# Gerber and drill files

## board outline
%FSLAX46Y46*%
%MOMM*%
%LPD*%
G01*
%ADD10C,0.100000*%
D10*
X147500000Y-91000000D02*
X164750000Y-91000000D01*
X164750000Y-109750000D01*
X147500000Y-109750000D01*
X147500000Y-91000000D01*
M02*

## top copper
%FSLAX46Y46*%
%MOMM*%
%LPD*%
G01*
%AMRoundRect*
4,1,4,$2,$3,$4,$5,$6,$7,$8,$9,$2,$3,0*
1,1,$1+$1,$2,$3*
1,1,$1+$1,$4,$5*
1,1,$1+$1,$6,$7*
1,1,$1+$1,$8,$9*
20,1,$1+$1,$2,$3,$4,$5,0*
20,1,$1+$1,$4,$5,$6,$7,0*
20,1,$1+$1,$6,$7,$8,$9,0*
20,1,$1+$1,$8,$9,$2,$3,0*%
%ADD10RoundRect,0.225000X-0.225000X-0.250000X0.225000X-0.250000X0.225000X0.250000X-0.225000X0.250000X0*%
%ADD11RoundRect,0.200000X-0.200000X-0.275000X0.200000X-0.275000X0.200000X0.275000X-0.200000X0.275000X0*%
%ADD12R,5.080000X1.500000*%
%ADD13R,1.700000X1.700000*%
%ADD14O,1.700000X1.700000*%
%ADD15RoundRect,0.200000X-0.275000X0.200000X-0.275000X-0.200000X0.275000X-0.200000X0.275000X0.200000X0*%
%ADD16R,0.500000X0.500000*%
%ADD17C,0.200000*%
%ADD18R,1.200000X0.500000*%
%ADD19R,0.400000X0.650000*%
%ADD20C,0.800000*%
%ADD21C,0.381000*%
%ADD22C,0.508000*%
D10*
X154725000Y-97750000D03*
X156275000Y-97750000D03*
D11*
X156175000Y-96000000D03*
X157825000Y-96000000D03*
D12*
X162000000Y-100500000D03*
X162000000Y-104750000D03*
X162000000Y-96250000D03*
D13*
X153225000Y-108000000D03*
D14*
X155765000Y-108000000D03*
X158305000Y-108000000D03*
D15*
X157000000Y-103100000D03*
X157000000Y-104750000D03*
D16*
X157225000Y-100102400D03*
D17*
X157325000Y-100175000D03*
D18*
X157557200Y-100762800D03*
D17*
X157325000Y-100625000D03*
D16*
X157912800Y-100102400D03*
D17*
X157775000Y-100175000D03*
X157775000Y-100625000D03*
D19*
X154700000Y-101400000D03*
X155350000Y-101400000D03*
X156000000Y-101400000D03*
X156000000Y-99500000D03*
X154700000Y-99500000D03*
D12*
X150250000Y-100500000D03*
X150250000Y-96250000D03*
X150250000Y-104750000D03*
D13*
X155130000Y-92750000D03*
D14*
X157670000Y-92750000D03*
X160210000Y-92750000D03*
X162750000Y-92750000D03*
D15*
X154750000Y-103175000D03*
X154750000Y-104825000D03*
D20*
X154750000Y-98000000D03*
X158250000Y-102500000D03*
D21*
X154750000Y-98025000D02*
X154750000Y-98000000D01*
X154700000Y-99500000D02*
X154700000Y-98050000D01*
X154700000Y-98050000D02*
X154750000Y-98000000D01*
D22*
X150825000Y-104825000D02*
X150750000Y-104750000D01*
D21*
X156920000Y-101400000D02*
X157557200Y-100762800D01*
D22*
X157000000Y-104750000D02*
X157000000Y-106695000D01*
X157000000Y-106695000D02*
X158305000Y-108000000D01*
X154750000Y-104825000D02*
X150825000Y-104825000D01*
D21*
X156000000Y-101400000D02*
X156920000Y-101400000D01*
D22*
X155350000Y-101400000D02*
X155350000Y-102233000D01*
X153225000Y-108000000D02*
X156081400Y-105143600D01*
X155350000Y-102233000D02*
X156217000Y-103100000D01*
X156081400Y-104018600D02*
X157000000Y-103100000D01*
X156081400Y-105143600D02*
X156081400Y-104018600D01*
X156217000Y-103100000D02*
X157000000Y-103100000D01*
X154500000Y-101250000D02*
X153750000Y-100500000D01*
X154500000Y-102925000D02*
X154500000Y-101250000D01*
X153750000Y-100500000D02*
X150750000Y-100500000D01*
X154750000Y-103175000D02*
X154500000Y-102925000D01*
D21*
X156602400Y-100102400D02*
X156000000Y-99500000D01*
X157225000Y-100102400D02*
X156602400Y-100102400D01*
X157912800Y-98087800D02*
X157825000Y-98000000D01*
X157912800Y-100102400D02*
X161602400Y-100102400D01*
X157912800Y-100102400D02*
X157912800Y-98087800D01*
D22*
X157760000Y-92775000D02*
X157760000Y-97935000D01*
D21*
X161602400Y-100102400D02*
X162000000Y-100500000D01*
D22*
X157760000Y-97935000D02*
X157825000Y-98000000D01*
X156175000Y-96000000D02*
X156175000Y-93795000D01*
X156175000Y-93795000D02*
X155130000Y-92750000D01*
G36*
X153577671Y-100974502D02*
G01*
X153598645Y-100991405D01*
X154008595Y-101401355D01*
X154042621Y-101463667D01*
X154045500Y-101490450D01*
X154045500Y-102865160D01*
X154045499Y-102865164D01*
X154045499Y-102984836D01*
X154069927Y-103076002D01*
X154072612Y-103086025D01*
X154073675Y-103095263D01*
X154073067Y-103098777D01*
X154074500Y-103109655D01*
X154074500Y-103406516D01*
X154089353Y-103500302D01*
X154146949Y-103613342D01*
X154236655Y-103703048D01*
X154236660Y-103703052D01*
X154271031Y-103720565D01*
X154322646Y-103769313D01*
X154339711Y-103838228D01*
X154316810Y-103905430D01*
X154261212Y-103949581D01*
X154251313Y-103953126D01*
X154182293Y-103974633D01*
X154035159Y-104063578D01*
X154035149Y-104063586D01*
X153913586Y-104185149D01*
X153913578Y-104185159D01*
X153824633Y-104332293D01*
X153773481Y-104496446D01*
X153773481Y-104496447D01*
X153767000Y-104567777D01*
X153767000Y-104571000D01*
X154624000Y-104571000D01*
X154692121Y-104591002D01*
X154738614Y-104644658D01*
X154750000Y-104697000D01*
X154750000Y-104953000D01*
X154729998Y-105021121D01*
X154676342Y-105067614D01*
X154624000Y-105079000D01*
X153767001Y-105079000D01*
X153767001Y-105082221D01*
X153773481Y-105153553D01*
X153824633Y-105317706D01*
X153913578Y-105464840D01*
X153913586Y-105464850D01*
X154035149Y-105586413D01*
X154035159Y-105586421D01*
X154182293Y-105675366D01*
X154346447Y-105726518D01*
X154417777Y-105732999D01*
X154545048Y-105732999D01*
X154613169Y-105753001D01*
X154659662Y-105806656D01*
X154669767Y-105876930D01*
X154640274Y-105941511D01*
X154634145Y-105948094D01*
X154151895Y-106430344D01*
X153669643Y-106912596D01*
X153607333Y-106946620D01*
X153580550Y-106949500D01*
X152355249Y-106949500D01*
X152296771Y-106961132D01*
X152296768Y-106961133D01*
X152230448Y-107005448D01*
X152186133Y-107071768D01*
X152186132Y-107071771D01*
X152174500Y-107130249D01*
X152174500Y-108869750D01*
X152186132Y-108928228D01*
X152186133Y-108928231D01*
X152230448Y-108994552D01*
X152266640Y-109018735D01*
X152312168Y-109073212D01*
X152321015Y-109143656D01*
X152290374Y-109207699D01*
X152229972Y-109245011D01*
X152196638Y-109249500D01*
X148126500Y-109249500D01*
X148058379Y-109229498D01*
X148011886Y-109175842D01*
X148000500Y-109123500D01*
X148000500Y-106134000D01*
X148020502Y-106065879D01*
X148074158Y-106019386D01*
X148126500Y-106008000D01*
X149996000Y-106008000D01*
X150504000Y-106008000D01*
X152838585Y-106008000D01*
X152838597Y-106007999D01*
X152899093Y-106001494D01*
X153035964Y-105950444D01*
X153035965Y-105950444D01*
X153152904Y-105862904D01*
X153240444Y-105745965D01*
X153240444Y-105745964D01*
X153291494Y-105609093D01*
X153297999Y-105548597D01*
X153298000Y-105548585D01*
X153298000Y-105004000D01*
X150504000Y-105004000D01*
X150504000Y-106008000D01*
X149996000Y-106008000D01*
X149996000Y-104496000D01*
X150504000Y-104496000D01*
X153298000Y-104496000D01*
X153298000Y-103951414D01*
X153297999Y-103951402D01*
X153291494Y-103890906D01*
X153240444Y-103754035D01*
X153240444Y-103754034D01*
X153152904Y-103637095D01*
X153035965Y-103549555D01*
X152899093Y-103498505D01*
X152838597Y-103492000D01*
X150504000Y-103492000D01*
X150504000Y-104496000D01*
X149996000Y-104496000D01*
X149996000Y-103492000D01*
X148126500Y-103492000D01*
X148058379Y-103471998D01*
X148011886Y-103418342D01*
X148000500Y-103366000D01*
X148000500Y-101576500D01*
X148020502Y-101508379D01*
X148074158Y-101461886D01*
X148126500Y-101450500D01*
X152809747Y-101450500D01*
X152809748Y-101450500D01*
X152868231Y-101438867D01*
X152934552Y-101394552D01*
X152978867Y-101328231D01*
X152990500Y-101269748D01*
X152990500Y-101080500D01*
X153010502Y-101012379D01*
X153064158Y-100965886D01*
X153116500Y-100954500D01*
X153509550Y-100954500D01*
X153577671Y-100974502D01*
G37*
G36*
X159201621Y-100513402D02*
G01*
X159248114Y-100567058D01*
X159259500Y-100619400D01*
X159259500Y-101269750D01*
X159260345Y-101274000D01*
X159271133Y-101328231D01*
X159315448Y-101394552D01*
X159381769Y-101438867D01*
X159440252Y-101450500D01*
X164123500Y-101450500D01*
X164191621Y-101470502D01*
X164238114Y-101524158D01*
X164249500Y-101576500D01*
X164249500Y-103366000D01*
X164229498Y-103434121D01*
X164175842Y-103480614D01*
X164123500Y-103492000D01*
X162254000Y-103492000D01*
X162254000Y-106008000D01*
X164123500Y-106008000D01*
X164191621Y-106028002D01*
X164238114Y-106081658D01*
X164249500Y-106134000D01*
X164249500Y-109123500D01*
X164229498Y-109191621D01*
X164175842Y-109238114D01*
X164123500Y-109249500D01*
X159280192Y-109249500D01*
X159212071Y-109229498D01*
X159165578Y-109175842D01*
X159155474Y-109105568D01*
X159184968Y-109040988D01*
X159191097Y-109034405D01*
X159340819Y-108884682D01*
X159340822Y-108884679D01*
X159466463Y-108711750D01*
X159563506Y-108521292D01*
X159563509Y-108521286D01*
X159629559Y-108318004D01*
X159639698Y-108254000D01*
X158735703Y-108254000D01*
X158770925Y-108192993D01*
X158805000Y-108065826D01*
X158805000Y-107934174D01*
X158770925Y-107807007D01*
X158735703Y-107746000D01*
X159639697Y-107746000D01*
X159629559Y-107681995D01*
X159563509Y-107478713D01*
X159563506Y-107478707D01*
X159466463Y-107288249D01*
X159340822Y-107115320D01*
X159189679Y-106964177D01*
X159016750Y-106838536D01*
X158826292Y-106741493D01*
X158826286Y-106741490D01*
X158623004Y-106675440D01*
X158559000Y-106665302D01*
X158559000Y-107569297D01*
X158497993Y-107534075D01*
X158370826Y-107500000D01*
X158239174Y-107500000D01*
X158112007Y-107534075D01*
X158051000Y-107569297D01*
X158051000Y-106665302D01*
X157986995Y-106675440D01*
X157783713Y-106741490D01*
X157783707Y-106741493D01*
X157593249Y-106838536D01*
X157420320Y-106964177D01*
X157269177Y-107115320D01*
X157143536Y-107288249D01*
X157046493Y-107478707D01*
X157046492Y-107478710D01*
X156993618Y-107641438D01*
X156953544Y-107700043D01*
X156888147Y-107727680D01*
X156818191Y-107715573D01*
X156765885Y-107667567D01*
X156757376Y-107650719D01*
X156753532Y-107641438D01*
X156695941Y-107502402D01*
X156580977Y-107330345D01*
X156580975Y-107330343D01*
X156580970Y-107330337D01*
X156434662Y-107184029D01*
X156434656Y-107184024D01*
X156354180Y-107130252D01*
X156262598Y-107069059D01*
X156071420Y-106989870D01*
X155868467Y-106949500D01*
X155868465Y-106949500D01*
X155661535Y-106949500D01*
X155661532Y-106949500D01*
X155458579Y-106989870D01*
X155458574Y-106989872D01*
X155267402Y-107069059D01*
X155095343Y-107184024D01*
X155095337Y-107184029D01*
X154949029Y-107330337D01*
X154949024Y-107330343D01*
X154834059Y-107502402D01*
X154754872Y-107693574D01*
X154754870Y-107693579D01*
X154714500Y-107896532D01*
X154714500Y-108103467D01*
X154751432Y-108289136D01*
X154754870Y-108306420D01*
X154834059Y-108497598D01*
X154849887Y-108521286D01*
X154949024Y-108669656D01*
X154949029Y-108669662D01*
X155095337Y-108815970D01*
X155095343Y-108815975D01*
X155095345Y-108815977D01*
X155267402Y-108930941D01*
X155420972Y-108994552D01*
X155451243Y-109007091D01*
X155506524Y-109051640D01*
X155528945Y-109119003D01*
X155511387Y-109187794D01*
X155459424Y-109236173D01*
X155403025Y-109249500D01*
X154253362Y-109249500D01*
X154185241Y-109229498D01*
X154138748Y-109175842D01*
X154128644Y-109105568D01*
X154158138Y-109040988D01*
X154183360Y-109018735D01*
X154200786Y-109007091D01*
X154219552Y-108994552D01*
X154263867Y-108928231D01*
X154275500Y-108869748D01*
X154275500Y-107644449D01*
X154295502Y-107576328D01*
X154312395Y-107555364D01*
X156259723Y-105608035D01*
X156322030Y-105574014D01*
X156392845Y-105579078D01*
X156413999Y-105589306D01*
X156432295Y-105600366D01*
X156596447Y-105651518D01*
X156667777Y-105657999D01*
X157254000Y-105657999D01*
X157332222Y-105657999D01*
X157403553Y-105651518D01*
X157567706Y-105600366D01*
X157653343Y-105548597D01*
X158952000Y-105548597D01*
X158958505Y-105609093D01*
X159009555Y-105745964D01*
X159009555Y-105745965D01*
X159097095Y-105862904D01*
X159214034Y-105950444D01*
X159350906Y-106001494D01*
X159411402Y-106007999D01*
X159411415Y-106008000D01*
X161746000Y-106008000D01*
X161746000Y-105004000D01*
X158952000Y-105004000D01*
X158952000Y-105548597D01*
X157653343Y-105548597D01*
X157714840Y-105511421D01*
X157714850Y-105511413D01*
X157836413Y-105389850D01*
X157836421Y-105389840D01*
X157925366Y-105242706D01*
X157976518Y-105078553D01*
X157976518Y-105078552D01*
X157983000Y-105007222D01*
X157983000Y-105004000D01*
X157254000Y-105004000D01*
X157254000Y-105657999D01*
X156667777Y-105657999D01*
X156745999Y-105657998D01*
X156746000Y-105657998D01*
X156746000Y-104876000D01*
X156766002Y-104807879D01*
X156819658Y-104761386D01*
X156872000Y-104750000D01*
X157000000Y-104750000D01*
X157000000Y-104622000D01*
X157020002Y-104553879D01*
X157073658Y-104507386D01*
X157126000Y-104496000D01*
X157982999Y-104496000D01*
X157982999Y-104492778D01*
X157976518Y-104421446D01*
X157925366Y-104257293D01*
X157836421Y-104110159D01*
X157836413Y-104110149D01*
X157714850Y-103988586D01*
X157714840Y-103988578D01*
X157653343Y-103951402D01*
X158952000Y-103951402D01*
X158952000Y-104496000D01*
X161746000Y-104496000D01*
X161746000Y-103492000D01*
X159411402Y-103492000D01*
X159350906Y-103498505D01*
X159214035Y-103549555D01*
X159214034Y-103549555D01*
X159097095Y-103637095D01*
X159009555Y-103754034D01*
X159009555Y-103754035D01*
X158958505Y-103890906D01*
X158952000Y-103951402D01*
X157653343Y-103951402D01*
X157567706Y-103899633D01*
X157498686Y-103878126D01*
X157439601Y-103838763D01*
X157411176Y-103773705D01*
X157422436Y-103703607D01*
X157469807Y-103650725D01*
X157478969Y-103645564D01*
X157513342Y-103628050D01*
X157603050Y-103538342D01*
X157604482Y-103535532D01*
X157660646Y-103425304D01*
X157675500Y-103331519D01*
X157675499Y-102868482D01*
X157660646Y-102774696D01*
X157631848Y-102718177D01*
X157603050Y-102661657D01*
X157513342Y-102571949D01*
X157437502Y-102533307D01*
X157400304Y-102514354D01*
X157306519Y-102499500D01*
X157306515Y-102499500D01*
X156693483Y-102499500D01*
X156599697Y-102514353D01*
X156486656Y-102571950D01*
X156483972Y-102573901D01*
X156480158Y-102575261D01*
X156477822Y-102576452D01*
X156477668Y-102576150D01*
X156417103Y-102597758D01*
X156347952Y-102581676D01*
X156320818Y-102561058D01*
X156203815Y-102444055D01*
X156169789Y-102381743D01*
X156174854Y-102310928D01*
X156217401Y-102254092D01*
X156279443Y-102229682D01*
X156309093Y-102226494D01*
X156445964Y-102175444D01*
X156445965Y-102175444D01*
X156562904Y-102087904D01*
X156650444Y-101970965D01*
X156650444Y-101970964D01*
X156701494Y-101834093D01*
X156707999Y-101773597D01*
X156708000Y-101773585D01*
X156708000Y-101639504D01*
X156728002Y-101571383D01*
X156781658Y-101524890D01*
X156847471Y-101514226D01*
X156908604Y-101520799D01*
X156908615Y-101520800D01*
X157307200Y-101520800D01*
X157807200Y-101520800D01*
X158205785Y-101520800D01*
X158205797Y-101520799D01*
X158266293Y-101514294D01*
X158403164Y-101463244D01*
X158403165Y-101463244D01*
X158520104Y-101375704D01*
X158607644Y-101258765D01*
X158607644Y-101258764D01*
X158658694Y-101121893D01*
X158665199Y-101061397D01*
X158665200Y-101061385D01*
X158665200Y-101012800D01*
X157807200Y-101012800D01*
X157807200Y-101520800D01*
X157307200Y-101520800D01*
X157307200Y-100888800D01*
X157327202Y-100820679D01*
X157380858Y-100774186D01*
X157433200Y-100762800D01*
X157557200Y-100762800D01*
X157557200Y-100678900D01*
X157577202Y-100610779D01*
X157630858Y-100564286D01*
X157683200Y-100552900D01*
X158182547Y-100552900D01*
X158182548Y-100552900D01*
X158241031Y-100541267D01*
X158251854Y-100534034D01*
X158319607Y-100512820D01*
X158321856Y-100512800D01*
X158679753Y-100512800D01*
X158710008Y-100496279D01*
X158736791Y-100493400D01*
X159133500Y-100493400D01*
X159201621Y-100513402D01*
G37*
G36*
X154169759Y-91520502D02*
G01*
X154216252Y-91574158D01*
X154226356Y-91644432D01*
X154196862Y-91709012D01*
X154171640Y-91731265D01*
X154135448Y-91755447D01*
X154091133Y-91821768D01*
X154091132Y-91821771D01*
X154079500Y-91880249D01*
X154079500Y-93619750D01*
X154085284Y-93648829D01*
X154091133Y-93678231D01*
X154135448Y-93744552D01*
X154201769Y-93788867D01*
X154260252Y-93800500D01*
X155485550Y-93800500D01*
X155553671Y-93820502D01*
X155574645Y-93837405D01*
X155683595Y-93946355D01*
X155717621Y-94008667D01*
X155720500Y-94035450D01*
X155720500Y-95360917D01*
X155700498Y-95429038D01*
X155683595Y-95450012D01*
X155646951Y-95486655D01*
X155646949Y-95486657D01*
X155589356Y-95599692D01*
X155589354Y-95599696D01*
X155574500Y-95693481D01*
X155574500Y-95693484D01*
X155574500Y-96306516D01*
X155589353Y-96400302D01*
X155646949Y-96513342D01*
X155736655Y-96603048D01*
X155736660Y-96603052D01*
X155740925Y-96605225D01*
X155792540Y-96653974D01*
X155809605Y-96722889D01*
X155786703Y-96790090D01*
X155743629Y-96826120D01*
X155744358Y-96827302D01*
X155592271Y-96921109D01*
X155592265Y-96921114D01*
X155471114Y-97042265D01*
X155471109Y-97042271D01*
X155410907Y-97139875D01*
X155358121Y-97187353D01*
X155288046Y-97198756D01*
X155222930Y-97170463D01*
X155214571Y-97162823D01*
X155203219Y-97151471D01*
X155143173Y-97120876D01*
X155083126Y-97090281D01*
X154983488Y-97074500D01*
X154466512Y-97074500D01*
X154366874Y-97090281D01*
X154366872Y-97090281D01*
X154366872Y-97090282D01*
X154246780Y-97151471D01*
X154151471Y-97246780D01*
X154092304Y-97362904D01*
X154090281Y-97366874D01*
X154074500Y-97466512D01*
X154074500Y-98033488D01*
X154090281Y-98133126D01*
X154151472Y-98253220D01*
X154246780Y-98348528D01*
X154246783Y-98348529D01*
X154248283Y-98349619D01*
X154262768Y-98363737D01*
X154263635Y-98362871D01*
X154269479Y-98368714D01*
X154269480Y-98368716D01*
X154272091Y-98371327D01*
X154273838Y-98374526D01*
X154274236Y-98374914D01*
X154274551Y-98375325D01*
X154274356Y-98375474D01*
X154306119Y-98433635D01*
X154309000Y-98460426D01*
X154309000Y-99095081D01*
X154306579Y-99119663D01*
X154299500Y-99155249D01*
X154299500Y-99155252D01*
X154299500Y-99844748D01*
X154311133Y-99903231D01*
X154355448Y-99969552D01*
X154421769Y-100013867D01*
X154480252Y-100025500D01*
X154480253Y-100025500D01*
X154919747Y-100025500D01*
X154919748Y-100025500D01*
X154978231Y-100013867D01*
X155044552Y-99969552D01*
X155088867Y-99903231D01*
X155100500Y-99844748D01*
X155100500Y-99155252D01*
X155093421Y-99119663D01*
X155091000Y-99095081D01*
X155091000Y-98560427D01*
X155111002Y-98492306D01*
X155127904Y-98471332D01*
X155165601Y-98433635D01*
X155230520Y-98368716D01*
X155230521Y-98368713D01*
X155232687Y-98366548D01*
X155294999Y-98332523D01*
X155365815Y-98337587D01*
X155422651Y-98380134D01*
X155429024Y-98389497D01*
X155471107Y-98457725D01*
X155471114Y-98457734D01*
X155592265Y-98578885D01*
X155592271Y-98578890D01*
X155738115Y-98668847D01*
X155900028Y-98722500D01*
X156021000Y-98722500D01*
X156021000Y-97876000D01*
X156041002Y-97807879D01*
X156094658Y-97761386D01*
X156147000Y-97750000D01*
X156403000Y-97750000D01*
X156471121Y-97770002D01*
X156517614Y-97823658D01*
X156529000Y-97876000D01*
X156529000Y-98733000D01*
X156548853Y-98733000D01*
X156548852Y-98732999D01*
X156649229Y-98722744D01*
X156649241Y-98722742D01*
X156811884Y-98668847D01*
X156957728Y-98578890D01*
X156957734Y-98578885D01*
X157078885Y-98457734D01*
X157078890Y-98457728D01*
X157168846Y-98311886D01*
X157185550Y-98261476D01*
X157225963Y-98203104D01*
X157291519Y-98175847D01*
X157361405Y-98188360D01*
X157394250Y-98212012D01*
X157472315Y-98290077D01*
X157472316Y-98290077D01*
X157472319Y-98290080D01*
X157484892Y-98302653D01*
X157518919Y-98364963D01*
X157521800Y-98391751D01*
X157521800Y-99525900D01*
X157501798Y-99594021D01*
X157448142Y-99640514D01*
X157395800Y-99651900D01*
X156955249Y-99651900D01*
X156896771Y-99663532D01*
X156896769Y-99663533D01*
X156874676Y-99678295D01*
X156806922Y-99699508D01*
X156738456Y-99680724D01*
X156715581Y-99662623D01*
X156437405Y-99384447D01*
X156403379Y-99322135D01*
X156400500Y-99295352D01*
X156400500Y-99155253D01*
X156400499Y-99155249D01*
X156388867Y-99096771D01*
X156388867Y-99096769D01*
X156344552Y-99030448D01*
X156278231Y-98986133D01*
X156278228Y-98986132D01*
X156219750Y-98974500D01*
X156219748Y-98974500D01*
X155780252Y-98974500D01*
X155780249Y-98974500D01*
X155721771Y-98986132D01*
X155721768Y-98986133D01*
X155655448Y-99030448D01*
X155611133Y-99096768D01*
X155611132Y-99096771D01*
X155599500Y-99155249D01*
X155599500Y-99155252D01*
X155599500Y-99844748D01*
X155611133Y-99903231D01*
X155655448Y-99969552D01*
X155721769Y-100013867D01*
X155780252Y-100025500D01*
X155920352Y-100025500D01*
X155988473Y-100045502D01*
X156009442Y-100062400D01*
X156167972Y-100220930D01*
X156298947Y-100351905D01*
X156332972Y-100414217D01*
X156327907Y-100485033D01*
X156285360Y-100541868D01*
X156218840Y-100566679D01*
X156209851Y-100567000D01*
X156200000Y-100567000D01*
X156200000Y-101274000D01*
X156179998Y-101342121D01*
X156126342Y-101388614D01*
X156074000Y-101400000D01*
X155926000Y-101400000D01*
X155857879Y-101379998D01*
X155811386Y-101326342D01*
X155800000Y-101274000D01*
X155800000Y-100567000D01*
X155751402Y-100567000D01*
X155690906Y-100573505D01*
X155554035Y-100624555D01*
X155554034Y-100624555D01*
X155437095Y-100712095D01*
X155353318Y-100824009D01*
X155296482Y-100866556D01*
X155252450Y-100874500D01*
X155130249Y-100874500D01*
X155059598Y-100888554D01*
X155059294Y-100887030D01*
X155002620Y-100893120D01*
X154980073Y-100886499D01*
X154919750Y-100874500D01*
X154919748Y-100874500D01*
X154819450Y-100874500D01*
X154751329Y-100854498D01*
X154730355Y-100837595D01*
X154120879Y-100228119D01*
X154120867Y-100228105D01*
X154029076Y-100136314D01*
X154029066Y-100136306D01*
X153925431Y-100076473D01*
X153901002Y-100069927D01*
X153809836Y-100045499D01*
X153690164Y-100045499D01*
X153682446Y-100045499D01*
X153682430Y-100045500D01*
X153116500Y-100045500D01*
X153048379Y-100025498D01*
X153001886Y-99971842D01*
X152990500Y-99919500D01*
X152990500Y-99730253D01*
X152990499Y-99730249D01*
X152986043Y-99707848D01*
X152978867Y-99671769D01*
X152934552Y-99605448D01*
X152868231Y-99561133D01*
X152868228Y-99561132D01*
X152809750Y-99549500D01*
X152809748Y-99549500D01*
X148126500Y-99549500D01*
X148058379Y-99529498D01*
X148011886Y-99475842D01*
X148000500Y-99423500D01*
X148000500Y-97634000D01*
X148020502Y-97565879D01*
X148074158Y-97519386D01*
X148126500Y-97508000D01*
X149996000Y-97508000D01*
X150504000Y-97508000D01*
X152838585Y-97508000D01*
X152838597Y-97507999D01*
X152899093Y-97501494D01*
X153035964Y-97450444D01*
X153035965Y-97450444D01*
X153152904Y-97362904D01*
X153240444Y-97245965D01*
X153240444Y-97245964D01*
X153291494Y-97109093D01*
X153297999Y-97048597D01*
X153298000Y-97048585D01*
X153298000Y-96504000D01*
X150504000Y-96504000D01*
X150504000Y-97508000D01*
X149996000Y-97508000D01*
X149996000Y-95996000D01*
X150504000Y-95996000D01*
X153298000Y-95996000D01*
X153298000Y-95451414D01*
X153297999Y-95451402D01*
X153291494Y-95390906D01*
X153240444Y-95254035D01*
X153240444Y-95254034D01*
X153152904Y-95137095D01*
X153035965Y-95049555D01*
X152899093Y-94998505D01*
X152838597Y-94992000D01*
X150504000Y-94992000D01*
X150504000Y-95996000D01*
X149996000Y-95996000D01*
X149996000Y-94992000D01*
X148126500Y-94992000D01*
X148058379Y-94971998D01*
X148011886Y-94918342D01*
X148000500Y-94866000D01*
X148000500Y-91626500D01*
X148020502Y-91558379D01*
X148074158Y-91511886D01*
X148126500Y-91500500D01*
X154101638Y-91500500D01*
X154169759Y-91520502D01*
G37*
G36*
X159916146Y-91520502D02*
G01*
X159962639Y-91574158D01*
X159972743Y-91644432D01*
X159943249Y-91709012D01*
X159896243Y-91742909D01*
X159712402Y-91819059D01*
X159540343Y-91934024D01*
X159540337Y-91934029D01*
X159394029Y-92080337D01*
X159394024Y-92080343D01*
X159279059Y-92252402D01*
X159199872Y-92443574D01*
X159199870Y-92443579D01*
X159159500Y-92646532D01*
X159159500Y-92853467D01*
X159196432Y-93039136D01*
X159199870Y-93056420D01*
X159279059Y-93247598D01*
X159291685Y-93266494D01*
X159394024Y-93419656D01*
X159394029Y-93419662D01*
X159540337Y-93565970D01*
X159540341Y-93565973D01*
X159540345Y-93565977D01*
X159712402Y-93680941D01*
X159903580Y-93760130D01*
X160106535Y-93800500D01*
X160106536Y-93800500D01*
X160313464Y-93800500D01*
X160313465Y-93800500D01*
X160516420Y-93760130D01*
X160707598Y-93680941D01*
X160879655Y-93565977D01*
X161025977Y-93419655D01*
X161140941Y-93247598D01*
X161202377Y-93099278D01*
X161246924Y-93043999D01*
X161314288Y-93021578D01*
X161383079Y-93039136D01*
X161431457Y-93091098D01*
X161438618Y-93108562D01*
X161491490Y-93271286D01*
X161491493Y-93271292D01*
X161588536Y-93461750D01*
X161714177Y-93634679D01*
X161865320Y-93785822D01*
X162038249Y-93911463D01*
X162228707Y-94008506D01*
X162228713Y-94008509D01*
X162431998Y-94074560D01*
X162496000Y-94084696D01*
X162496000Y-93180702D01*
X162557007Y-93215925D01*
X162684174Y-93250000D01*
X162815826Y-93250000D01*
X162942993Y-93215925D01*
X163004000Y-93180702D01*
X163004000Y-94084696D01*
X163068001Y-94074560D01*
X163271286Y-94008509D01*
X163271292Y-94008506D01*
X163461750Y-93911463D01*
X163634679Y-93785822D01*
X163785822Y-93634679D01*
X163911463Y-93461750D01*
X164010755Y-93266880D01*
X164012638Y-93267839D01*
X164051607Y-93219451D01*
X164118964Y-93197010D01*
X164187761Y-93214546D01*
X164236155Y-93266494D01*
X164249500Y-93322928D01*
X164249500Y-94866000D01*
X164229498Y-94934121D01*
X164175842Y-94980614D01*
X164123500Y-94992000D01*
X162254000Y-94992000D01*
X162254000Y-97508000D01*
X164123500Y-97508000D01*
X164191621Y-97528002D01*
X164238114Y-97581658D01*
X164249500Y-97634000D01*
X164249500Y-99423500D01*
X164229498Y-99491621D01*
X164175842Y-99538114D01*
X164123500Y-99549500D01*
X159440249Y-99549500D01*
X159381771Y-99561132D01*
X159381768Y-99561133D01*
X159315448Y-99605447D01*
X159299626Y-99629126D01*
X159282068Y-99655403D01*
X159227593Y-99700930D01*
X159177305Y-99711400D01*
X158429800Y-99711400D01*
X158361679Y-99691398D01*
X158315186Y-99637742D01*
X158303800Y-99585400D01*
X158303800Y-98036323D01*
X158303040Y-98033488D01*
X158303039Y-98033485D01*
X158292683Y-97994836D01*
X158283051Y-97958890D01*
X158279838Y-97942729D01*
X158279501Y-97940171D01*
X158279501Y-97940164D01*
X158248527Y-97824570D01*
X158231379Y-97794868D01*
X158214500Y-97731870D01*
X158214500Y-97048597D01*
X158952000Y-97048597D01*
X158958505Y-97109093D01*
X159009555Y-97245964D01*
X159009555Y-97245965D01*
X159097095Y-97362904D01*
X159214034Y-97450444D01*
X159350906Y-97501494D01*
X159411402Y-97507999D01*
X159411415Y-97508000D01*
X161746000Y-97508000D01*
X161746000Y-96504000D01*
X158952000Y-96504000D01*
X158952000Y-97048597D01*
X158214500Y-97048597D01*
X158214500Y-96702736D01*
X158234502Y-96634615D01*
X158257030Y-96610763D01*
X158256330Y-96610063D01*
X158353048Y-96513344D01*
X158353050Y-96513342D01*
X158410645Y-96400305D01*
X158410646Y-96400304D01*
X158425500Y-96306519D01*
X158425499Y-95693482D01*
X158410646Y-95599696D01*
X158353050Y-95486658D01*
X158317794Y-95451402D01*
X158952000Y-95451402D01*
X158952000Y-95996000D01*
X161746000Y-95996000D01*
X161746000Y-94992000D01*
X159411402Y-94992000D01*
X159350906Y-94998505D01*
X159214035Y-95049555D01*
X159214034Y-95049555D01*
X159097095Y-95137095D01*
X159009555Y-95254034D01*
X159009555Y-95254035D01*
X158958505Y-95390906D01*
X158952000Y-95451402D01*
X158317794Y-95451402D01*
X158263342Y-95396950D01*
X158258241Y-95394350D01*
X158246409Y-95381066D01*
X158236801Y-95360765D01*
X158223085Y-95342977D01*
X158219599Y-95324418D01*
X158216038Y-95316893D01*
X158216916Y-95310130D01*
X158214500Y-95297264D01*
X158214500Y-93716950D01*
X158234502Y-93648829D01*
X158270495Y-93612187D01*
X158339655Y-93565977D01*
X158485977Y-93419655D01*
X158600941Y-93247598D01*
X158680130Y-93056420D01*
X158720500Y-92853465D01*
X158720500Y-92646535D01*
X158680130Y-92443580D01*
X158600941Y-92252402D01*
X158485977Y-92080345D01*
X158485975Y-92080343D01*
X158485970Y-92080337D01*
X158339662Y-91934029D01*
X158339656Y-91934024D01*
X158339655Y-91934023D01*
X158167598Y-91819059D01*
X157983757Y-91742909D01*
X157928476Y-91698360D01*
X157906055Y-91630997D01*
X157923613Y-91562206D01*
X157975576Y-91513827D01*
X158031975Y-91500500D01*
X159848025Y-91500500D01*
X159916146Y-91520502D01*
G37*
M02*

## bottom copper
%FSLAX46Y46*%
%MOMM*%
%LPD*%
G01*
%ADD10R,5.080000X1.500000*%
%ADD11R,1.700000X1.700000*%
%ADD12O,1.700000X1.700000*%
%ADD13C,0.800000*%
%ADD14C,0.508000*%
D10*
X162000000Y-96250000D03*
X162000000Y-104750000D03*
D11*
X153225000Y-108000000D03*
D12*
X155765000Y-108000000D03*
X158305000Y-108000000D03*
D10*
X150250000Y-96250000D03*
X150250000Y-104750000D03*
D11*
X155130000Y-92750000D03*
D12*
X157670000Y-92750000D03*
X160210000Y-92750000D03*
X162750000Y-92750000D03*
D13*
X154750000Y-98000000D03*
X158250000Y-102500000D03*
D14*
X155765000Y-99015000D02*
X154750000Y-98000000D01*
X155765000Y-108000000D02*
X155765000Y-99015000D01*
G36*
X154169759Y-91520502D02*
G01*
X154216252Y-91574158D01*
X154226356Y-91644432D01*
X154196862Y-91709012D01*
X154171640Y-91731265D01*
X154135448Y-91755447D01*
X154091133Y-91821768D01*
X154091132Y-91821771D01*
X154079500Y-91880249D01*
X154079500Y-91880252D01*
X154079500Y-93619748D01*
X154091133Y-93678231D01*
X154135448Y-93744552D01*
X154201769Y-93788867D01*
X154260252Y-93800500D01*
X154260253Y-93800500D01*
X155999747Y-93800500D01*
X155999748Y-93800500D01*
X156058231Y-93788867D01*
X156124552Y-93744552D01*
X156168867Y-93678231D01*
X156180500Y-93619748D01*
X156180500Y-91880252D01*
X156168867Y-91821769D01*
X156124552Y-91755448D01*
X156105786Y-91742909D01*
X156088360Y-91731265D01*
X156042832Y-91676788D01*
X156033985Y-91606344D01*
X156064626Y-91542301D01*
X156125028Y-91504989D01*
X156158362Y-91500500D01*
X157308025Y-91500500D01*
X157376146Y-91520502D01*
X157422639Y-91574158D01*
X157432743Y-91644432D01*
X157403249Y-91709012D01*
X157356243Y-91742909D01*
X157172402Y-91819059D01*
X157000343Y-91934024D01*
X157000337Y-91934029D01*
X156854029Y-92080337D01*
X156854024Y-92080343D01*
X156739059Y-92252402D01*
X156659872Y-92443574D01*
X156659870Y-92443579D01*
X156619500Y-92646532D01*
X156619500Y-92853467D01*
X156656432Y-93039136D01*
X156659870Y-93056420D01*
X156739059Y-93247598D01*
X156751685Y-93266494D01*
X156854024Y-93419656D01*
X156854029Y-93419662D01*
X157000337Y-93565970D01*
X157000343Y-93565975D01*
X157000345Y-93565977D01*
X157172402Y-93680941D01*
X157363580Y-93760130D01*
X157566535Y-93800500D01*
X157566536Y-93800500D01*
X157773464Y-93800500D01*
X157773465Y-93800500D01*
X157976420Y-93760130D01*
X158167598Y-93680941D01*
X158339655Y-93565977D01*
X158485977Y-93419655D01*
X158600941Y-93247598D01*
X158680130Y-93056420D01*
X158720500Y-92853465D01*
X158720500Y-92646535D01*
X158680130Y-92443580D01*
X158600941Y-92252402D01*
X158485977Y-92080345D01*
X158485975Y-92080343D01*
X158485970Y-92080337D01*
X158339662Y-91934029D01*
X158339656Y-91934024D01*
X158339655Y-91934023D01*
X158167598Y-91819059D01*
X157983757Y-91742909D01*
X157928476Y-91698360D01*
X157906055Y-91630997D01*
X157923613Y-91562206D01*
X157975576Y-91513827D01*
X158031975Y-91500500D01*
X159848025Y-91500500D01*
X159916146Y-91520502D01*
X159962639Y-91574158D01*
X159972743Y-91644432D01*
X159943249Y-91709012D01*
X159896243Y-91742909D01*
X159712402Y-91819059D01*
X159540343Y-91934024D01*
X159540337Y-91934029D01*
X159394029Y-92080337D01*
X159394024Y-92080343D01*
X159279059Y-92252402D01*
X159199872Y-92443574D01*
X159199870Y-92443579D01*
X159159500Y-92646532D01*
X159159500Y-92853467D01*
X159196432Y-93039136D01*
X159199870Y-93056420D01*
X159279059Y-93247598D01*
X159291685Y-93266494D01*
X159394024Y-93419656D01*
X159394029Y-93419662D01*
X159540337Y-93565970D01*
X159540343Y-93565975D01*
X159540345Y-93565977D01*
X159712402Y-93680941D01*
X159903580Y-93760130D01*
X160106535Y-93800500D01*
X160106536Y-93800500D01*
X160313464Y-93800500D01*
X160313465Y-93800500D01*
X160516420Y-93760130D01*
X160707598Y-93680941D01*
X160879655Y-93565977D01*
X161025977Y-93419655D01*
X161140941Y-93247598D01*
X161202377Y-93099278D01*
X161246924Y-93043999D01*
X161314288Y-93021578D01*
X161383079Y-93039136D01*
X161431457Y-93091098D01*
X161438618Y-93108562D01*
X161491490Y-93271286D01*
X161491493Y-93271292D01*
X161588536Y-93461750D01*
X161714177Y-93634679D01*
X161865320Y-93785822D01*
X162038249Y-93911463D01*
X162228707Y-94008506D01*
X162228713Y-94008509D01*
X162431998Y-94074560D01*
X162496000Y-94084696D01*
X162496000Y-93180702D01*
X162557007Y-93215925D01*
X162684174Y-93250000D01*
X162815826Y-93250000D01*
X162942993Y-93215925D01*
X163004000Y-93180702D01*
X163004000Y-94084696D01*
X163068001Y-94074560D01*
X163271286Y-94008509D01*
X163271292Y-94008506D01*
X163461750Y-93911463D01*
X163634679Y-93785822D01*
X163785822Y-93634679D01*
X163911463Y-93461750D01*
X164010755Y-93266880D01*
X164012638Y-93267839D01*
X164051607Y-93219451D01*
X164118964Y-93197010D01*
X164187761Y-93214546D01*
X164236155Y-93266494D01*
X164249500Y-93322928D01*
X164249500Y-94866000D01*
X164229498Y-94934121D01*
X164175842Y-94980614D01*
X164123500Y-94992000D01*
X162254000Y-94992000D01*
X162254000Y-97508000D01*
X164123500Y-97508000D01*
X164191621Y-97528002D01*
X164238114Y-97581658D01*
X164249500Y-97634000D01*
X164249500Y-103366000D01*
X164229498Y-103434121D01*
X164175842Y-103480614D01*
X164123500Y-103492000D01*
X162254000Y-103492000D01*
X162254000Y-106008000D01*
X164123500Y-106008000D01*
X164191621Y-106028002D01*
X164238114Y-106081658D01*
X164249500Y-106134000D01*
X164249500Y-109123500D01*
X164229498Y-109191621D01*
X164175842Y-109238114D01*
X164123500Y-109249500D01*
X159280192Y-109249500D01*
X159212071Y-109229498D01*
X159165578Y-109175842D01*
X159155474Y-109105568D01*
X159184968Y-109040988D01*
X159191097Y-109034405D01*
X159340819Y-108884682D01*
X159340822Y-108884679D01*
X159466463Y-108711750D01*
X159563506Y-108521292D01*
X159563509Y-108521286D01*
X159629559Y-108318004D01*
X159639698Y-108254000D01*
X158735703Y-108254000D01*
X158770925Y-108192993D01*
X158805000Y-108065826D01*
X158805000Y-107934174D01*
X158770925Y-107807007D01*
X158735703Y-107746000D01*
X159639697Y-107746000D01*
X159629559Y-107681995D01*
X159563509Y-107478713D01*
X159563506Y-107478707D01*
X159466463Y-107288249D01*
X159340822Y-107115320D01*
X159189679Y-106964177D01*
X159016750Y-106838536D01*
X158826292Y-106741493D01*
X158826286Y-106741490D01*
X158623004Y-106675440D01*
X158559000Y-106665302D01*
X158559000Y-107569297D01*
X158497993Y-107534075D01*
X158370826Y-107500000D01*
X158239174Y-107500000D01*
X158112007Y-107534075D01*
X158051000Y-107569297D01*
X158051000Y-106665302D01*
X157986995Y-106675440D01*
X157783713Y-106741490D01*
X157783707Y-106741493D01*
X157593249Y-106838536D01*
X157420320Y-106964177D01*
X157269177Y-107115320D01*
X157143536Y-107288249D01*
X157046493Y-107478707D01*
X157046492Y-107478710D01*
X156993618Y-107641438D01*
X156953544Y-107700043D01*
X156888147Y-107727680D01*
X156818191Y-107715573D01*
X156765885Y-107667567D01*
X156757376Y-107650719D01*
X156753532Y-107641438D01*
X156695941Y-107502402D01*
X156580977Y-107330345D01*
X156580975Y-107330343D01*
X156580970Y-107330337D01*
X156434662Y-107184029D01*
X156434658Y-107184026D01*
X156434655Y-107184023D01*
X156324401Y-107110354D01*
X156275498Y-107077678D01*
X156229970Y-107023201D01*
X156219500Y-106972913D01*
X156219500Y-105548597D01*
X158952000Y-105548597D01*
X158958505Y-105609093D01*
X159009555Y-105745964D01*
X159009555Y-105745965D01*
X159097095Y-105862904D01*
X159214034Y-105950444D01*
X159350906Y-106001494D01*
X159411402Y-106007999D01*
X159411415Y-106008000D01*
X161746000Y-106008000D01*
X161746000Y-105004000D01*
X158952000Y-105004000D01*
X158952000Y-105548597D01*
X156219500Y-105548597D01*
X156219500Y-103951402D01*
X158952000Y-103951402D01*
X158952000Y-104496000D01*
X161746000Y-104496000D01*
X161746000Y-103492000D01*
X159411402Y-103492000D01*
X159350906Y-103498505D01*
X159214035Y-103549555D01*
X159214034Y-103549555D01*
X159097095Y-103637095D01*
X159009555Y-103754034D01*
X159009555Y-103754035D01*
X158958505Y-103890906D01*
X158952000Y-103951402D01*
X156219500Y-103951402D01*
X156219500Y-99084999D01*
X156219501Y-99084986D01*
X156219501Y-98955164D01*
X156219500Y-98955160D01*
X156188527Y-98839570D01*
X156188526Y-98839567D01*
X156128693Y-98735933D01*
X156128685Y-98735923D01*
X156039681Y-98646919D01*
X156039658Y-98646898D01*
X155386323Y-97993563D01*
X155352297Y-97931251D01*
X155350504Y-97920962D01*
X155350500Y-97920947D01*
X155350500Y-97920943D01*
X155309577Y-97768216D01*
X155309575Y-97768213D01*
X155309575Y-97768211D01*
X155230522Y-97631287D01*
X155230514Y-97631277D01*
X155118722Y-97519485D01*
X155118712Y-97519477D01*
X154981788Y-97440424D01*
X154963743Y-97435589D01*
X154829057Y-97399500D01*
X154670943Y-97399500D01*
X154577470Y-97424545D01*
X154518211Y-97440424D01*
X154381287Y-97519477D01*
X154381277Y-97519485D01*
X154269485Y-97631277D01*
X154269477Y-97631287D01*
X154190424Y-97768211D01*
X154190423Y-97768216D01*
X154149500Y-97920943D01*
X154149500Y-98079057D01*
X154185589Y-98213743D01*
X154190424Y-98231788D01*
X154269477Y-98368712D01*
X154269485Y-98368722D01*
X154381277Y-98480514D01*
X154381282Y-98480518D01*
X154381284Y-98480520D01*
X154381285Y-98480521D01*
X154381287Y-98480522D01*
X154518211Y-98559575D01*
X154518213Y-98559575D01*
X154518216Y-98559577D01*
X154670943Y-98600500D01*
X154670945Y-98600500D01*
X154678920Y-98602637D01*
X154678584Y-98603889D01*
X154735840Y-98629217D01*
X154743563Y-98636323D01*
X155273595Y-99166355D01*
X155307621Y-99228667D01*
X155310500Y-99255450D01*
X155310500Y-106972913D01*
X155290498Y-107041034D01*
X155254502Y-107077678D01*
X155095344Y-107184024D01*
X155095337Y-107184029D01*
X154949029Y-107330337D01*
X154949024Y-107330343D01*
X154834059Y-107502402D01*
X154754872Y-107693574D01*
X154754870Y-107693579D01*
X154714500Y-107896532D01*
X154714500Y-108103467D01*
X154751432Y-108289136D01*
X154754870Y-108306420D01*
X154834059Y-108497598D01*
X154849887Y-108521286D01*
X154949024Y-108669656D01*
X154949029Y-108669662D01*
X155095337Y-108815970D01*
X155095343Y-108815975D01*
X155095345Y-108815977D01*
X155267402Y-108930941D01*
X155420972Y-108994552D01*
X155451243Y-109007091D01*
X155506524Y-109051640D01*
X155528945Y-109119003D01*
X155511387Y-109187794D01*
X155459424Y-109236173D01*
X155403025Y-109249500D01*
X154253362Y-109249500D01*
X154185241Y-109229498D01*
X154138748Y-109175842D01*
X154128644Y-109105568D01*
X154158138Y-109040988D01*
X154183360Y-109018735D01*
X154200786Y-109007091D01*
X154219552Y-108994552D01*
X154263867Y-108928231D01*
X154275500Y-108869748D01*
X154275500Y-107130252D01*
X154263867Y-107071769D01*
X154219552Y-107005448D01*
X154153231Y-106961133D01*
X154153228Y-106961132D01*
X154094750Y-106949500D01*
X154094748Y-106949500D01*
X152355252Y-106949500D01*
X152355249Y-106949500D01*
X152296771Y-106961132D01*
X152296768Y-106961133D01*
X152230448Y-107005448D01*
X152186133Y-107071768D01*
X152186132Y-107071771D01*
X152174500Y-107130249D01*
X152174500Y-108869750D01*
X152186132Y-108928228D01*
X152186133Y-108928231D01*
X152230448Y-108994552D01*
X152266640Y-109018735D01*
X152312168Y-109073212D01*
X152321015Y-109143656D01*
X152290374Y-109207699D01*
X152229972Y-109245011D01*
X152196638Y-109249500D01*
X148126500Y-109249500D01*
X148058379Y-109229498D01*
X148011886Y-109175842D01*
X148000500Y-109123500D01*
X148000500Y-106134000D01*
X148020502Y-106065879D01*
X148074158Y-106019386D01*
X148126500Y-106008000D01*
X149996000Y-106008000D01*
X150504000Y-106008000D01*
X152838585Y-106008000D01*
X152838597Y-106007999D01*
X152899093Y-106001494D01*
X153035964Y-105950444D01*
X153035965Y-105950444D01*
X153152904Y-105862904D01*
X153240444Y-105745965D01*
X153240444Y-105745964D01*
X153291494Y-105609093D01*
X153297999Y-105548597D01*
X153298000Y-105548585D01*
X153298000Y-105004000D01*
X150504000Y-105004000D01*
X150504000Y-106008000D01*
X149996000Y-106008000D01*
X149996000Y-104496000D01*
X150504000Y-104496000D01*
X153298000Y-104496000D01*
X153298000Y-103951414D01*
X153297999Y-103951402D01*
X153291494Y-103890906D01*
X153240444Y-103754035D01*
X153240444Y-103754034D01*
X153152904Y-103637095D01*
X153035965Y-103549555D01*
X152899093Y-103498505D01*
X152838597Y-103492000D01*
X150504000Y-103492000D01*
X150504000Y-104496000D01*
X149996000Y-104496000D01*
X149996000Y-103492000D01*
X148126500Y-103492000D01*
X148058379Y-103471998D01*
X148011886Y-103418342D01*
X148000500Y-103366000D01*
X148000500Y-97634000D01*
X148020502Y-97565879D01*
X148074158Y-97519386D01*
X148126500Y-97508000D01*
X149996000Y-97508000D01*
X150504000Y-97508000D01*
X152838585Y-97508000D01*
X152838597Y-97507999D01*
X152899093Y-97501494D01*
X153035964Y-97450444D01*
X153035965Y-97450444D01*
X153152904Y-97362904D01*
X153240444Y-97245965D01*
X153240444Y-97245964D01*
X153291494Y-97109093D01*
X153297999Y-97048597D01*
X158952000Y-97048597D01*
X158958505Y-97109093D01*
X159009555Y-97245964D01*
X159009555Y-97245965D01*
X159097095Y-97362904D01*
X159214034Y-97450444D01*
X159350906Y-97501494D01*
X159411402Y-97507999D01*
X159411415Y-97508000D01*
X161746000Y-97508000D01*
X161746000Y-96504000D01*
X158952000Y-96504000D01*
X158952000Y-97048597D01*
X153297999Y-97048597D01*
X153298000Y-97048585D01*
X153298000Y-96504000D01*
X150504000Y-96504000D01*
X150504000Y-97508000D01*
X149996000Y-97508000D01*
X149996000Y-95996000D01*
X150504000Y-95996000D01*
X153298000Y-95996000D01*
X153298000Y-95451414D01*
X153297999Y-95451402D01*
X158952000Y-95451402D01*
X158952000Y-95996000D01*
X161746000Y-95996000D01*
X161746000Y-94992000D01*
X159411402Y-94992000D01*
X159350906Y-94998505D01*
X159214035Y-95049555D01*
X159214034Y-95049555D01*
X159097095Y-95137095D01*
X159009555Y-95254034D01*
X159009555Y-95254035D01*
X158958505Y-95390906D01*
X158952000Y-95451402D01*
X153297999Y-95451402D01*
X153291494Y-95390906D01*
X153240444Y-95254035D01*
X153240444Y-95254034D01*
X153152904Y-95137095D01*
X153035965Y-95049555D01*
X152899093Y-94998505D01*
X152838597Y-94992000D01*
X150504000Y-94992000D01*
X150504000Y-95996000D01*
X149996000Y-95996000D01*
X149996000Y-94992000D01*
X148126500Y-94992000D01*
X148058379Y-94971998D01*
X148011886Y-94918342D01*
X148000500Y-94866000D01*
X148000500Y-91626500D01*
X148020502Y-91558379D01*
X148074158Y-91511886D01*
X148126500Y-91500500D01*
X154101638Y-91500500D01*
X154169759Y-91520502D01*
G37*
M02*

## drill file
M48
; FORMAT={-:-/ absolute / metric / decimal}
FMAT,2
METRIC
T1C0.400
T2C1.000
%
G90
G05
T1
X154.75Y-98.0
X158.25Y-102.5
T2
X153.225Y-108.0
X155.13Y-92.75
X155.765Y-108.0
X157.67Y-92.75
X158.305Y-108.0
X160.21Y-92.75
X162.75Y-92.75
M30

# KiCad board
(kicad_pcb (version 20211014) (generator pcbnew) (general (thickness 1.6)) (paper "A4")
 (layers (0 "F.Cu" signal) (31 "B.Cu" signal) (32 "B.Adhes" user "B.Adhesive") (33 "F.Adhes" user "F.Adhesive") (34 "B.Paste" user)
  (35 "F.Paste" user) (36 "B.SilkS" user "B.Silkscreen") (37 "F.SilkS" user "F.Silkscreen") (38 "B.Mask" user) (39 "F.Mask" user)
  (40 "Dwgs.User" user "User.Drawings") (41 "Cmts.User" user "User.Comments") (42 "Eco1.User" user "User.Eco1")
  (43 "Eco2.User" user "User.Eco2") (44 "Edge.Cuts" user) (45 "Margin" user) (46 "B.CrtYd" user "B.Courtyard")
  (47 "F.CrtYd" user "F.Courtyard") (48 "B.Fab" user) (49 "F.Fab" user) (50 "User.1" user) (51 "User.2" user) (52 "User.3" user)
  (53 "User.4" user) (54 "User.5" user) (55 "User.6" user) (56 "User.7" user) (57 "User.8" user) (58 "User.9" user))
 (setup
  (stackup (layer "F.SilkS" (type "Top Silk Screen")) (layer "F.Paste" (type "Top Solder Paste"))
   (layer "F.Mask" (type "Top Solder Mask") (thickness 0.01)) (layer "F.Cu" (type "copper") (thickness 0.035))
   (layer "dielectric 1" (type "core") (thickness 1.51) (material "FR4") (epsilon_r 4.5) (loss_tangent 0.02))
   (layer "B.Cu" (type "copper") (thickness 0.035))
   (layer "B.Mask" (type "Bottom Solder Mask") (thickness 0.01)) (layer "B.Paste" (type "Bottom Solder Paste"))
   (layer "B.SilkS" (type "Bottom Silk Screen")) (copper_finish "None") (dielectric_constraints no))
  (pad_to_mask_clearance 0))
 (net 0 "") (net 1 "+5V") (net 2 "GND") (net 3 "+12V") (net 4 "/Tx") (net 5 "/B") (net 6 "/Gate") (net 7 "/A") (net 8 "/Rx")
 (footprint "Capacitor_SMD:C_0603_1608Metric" (layer "F.Cu") (at 155.5 97.75)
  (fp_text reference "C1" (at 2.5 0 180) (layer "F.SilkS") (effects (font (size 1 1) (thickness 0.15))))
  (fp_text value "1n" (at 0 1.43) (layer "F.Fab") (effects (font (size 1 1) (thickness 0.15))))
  (pad "1" smd roundrect (at -0.775 0) (size 0.9 0.95) (layers "F.Cu" "F.Paste" "F.Mask") (roundrect_rratio 0.25) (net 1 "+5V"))
  (pad "2" smd roundrect (at 0.775 0) (size 0.9 0.95) (layers "F.Cu" "F.Paste" "F.Mask") (roundrect_rratio 0.25) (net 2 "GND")))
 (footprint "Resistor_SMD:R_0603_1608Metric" (layer "F.Cu") (at 157 96)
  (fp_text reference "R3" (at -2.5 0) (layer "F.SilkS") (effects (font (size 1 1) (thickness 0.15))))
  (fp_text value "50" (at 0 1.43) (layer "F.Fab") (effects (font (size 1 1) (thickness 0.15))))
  (pad "1" smd roundrect (at -0.825 0) (size 0.8 0.95) (layers "F.Cu" "F.Paste" "F.Mask") (roundrect_rratio 0.25) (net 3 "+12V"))
  (pad "2" smd roundrect (at 0.825 0) (size 0.8 0.95) (layers "F.Cu" "F.Paste" "F.Mask") (roundrect_rratio 0.25) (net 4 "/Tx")))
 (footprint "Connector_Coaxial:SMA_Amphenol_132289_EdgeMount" (layer "F.Cu") (at 162 100.5)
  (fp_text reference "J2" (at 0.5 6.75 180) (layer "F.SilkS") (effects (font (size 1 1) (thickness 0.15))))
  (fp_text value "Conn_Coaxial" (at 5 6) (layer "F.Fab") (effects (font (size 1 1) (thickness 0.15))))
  (pad "1" smd rect (at 0 0 90) (size 1.5 5.08) (layers "F.Cu" "F.Paste" "F.Mask") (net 4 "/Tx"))
  (pad "2" smd rect (at 0 -4.25 90) (size 1.5 5.08) (layers "B.Cu" "B.Paste" "B.Mask") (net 2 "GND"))
  (pad "2" smd rect (at 0 4.25 90) (size 1.5 5.08) (layers "F.Cu" "F.Paste" "F.Mask") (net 2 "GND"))
  (pad "2" smd rect (at 0 4.25 90) (size 1.5 5.08) (layers "B.Cu" "B.Paste" "B.Mask") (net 2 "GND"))
  (pad "2" smd rect (at 0 -4.25 90) (size 1.5 5.08) (layers "F.Cu" "F.Paste" "F.Mask") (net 2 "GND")))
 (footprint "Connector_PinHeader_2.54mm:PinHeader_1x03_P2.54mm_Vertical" (layer "F.Cu") (at 153.225 108 90)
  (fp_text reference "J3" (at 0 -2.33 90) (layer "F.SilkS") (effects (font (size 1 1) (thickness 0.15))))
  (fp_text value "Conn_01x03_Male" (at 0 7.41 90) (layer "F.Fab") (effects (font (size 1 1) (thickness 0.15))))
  (pad "1" thru_hole rect (at 0 0 90) (size 1.7 1.7) (drill 1) (layers *.Cu *.Mask) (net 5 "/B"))
  (pad "2" thru_hole oval (at 0 2.54 90) (size 1.7 1.7) (drill 1) (layers *.Cu *.Mask) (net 1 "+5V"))
  (pad "3" thru_hole oval (at 0 5.08 90) (size 1.7 1.7) (drill 1) (layers *.Cu *.Mask) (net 2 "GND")))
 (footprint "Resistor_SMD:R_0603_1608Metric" (layer "F.Cu") (at 157 103.925 -90)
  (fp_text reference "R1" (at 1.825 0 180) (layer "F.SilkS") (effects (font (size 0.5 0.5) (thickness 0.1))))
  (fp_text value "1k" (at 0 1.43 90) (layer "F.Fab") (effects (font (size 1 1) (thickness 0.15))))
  (pad "1" smd roundrect (at -0.825 0 270) (size 0.8 0.95) (layers "F.Cu" "F.Paste" "F.Mask") (roundrect_rratio 0.25) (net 5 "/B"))
  (pad "2" smd roundrect (at 0.825 0 270) (size 0.8 0.95) (layers "F.Cu" "F.Paste" "F.Mask") (roundrect_rratio 0.25) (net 2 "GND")))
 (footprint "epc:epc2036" (layer "F.Cu") (at 157.1 99.95)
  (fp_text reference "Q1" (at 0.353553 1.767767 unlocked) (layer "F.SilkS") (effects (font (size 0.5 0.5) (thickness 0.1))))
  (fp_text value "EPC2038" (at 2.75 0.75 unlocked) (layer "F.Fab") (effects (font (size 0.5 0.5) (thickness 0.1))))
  (pad "1" smd rect (at 0.125 0.1524) (size 0.5 0.5) (layers "F.Cu") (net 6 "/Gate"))
  (pad "1" smd circle (at 0.225 0.225) (size 0.2 0.2) (layers "F.Cu" "F.Paste" "F.Mask") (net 6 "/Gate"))
  (pad "2" smd rect (at 0.4572 0.8128) (size 1.2 0.5) (layers "F.Cu") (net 2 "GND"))
  (pad "2" smd circle (at 0.225 0.675) (size 0.2 0.2) (layers "F.Cu" "F.Paste" "F.Mask") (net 2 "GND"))
  (pad "3" smd rect (at 0.8128 0.1524) (size 0.5 0.5) (layers "F.Cu") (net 4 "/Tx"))
  (pad "3" smd circle (at 0.675 0.225) (size 0.2 0.2) (layers "F.Cu" "F.Paste" "F.Mask") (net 4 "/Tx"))
  (pad "4" smd circle (at 0.675 0.675) (size 0.2 0.2) (layers "F.Cu" "F.Paste" "F.Mask") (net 2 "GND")))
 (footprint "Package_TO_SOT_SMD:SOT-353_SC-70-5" (layer "F.Cu") (at 155.35 100.45 90)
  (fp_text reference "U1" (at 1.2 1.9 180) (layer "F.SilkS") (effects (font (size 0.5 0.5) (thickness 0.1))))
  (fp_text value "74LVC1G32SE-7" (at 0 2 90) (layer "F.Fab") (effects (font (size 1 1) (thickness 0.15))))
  (pad "1" smd rect (at -0.95 -0.65 90) (size 0.65 0.4) (layers "F.Cu" "F.Paste" "F.Mask") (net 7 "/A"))
  (pad "2" smd rect (at -0.95 0 90) (size 0.65 0.4) (layers "F.Cu" "F.Paste" "F.Mask") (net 5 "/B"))
  (pad "3" smd rect (at -0.95 0.65 90) (size 0.65 0.4) (layers "F.Cu" "F.Paste" "F.Mask") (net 2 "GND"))
  (pad "4" smd rect (at 0.95 0.65 90) (size 0.65 0.4) (layers "F.Cu" "F.Paste" "F.Mask") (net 6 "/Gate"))
  (pad "5" smd rect (at 0.95 -0.65 90) (size 0.65 0.4) (layers "F.Cu" "F.Paste" "F.Mask") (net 1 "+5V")))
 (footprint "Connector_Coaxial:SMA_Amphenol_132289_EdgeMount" (layer "F.Cu") (at 150.25 100.5 180)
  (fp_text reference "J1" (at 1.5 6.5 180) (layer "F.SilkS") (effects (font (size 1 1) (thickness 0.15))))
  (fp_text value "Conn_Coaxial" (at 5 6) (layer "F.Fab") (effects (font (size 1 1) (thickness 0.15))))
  (pad "1" smd rect (at 0 0 270) (size 1.5 5.08) (layers "F.Cu" "F.Paste" "F.Mask") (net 7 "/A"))
  (pad "2" smd rect (at 0 4.25 270) (size 1.5 5.08) (layers "F.Cu" "F.Paste" "F.Mask") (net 2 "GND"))
  (pad "2" smd rect (at 0 4.25 270) (size 1.5 5.08) (layers "B.Cu" "B.Paste" "B.Mask") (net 2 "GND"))
  (pad "2" smd rect (at 0 -4.25 270) (size 1.5 5.08) (layers "F.Cu" "F.Paste" "F.Mask") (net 2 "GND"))
  (pad "2" smd rect (at 0 -4.25 270) (size 1.5 5.08) (layers "B.Cu" "B.Paste" "B.Mask") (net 2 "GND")))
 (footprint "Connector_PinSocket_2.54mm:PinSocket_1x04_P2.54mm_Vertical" (layer "F.Cu") (at 155.13 92.75 90)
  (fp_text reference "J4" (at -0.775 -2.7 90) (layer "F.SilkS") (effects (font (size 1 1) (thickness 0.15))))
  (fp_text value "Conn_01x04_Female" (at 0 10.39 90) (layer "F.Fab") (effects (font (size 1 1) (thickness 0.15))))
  (pad "1" thru_hole rect (at 0 0 90) (size 1.7 1.7) (drill 1) (layers *.Cu *.Mask) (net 3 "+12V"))
  (pad "2" thru_hole oval (at 0 2.54 90) (size 1.7 1.7) (drill 1) (layers *.Cu *.Mask) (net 4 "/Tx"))
  (pad "3" thru_hole oval (at 0 5.08 90) (size 1.7 1.7) (drill 1) (layers *.Cu *.Mask) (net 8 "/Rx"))
  (pad "4" thru_hole oval (at 0 7.62 90) (size 1.7 1.7) (drill 1) (layers *.Cu *.Mask) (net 2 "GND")))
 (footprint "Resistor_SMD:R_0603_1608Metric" (layer "F.Cu") (at 154.75 104 -90)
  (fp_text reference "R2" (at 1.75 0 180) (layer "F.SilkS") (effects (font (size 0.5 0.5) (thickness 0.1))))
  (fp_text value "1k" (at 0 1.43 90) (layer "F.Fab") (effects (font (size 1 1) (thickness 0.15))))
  (pad "1" smd roundrect (at -0.825 0 270) (size 0.8 0.95) (layers "F.Cu" "F.Paste" "F.Mask") (roundrect_rratio 0.25) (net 7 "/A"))
  (pad "2" smd roundrect (at 0.825 0 270) (size 0.8 0.95) (layers "F.Cu" "F.Paste" "F.Mask") (roundrect_rratio 0.25) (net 2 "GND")))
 (gr_rect (start 164.75 91) (end 147.5 109.75) (layer "Edge.Cuts") (width 0.1) (fill none))
 (segment (start 154.75 98.025) (end 154.75 98) (width 0.381) (layer "F.Cu") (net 1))
 (segment (start 154.7 99.5) (end 154.7 98.05) (width 0.381) (layer "F.Cu") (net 1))
 (segment (start 154.7 98.05) (end 154.75 98) (width 0.381) (layer "F.Cu") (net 1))
 (via (at 154.75 98) (size 0.8) (drill 0.4) (layers "F.Cu" "B.Cu") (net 1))
 (segment (start 155.765 99.015) (end 154.75 98) (width 0.508) (layer "B.Cu") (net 1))
 (segment (start 155.765 108) (end 155.765 99.015) (width 0.508) (layer "B.Cu") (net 1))
 (segment (start 150.825 104.825) (end 150.75 104.75) (width 0.508) (layer "F.Cu") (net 2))
 (segment (start 156.92 101.4) (end 157.5572 100.7628) (width 0.381) (layer "F.Cu") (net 2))
 (segment (start 157 104.75) (end 157 106.695) (width 0.508) (layer "F.Cu") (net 2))
 (segment (start 157 106.695) (end 158.305 108) (width 0.508) (layer "F.Cu") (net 2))
 (segment (start 154.75 104.825) (end 150.825 104.825) (width 0.508) (layer "F.Cu") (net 2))
 (segment (start 156 101.4) (end 156.92 101.4) (width 0.381) (layer "F.Cu") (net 2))
 (via (at 158.25 102.5) (size 0.8) (drill 0.4) (layers "F.Cu" "B.Cu") (free) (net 2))
 (segment (start 155.35 101.4) (end 155.35 102.233) (width 0.508) (layer "F.Cu") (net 5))
 (segment (start 153.225 108) (end 156.0814 105.1436) (width 0.508) (layer "F.Cu") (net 5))
 (segment (start 155.35 102.233) (end 156.217 103.1) (width 0.508) (layer "F.Cu") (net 5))
 (segment (start 156.0814 104.0186) (end 157 103.1) (width 0.508) (layer "F.Cu") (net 5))
 (segment (start 156.0814 105.1436) (end 156.0814 104.0186) (width 0.508) (layer "F.Cu") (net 5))
 (segment (start 156.217 103.1) (end 157 103.1) (width 0.508) (layer "F.Cu") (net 5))
 (segment (start 154.5 101.25) (end 153.75 100.5) (width 0.508) (layer "F.Cu") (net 7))
 (segment (start 154.5 102.925) (end 154.5 101.25) (width 0.508) (layer "F.Cu") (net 7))
 (segment (start 153.75 100.5) (end 150.75 100.5) (width 0.508) (layer "F.Cu") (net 7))
 (segment (start 154.75 103.175) (end 154.5 102.925) (width 0.508) (layer "F.Cu") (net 7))
 (segment (start 156.6024 100.1024) (end 156 99.5) (width 0.381) (layer "F.Cu") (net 6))
 (segment (start 157.225 100.1024) (end 156.6024 100.1024) (width 0.381) (layer "F.Cu") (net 6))
 (segment (start 157.9128 98.0878) (end 157.825 98) (width 0.381) (layer "F.Cu") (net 4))
 (segment (start 157.9128 100.1024) (end 161.6024 100.1024) (width 0.381) (layer "F.Cu") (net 4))
 (segment (start 157.9128 100.1024) (end 157.9128 98.0878) (width 0.381) (layer "F.Cu") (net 4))
 (segment (start 157.76 92.775) (end 157.76 97.935) (width 0.508) (layer "F.Cu") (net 4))
 (segment (start 161.6024 100.1024) (end 162 100.5) (width 0.381) (layer "F.Cu") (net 4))
 (segment (start 157.76 97.935) (end 157.825 98) (width 0.508) (layer "F.Cu") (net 4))
 (segment (start 156.175 96) (end 156.175 93.795) (width 0.508) (layer "F.Cu") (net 3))
 (segment (start 156.175 93.795) (end 155.13 92.75) (width 0.508) (layer "F.Cu") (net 3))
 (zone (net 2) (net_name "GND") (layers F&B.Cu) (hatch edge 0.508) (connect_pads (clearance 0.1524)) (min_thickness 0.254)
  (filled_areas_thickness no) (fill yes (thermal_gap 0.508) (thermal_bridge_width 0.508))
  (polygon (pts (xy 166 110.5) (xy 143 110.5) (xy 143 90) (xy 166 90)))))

